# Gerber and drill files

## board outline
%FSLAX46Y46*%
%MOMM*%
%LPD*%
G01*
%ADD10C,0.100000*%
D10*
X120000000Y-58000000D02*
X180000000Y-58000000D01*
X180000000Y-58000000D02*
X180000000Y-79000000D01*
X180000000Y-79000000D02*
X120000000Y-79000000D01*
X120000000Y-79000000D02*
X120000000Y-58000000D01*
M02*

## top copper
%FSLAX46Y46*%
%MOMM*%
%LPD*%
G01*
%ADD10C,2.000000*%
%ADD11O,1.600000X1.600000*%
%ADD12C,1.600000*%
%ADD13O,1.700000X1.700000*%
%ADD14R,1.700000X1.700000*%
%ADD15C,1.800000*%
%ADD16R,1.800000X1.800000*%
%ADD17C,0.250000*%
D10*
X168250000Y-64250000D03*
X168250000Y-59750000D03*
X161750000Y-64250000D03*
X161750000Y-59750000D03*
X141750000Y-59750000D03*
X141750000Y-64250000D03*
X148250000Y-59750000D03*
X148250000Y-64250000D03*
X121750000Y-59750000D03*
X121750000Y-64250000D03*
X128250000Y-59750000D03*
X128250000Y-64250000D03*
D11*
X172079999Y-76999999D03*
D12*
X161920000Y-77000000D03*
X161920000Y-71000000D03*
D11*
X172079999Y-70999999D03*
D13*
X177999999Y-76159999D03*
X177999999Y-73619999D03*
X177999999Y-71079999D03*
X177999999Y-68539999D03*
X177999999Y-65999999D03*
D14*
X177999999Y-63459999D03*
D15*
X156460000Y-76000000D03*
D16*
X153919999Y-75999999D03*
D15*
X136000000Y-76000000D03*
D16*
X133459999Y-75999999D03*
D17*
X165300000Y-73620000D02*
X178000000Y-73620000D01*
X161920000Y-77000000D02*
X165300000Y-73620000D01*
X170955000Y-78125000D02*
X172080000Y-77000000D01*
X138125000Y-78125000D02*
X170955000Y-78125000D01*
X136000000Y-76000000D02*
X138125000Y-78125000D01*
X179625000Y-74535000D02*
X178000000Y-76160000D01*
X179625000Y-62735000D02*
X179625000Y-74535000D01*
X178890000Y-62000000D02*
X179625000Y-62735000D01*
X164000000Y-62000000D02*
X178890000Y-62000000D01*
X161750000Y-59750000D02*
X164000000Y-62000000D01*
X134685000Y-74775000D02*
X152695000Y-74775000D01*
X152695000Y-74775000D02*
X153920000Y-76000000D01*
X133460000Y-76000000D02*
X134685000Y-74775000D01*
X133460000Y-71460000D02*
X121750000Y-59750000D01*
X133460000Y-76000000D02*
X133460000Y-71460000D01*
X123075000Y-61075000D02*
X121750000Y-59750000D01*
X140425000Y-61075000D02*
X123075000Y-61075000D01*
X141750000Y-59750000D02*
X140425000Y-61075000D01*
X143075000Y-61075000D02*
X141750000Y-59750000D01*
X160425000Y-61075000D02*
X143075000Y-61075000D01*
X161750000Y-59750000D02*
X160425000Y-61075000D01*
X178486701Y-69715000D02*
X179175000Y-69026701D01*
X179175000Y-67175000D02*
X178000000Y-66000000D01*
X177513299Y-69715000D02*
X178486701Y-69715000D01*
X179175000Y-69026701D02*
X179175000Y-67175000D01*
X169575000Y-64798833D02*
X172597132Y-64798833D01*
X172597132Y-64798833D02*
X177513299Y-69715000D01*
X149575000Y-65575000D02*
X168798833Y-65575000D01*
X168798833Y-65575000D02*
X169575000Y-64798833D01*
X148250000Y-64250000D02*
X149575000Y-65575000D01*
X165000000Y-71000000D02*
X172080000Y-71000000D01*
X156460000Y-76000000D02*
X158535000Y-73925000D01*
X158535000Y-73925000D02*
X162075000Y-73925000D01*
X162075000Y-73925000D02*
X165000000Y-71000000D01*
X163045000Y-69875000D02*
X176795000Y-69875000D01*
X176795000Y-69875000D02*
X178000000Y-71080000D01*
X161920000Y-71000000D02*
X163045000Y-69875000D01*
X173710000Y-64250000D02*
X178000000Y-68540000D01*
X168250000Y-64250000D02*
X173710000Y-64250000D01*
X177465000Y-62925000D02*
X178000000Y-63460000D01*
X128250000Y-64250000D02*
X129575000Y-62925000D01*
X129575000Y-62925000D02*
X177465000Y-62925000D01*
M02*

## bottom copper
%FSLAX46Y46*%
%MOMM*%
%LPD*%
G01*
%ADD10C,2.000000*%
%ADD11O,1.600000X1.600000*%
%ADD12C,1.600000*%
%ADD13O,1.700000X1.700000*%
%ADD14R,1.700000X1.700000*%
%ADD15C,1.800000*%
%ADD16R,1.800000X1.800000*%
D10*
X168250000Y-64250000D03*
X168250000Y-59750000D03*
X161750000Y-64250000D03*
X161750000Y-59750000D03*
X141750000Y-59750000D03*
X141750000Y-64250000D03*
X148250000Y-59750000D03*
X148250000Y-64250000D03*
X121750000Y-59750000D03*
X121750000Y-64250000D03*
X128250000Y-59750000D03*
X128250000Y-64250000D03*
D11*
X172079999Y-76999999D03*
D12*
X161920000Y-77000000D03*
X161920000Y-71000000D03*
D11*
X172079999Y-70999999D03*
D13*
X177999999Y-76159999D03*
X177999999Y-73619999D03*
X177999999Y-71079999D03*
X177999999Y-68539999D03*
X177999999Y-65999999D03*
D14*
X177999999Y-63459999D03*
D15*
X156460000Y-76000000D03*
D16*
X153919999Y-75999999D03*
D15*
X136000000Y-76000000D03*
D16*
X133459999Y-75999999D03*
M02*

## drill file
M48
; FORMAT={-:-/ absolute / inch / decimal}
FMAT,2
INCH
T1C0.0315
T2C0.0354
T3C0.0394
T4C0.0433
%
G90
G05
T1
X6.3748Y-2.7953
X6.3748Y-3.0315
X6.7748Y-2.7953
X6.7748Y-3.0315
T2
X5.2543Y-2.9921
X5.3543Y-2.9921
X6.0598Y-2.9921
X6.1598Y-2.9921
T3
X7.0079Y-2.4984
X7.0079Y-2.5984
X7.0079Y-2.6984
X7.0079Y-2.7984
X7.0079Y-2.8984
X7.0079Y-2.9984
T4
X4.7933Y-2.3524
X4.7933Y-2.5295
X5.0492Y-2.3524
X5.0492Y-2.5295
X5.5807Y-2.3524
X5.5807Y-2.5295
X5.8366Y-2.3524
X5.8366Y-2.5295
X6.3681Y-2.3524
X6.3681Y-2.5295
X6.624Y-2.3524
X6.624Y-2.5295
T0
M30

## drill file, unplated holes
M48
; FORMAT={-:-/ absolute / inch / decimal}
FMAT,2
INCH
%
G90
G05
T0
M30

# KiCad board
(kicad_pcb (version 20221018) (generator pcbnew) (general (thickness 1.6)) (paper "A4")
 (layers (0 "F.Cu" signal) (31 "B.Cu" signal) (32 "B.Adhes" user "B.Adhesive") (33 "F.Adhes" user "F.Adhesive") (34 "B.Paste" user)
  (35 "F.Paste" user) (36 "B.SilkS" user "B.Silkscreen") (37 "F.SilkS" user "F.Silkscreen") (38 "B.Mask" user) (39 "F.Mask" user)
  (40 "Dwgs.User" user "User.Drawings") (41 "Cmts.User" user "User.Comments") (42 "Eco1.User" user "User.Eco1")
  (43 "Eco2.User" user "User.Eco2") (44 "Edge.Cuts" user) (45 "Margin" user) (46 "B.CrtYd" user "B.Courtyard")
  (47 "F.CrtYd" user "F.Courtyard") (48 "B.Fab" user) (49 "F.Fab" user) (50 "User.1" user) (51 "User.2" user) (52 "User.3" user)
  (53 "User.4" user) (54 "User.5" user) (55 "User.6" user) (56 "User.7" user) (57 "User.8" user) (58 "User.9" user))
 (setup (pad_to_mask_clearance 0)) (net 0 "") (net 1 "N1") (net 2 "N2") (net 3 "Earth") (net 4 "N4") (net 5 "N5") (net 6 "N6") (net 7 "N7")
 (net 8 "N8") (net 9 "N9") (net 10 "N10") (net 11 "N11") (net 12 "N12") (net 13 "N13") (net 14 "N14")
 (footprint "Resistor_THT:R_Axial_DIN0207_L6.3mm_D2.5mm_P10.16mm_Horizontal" (layer "F.Cu") (at 161.92 77)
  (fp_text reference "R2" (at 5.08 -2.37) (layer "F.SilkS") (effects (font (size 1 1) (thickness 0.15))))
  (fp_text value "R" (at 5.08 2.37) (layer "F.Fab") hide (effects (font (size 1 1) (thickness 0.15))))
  (pad "1" thru_hole circle (at 0 0) (size 1.6 1.6) (drill 0.8) (layers "*.Cu" "*.Mask") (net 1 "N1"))
  (pad "2" thru_hole oval (at 10.16 0) (size 1.6 1.6) (drill 0.8) (layers "*.Cu" "*.Mask") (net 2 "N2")))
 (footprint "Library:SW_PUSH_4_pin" (layer "F.Cu") (at 161.75 59.75)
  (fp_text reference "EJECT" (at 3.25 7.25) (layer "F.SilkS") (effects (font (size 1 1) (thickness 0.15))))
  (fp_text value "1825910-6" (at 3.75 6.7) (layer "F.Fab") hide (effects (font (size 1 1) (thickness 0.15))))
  (pad "1" thru_hole circle (at 0 0 90) (size 2 2) (drill 1.1) (layers "*.Cu" "*.Mask") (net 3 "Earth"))
  (pad "2" thru_hole circle (at 0 4.5 90) (size 2 2) (drill 1.1) (layers "*.Cu" "*.Mask") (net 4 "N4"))
  (pad "3" thru_hole circle (at 6.5 0 90) (size 2 2) (drill 1.1) (layers "*.Cu" "*.Mask") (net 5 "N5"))
  (pad "4" thru_hole circle (at 6.5 4.5 90) (size 2 2) (drill 1.1) (layers "*.Cu" "*.Mask") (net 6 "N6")))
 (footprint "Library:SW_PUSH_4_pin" (layer "F.Cu") (at 141.75 59.75)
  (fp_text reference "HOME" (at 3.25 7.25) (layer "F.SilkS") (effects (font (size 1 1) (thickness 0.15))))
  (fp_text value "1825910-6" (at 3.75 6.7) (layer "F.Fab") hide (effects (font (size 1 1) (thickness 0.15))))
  (pad "1" thru_hole circle (at 0 0 90) (size 2 2) (drill 1.1) (layers "*.Cu" "*.Mask") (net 3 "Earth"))
  (pad "2" thru_hole circle (at 0 4.5 90) (size 2 2) (drill 1.1) (layers "*.Cu" "*.Mask") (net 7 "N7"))
  (pad "3" thru_hole circle (at 6.5 0 90) (size 2 2) (drill 1.1) (layers "*.Cu" "*.Mask") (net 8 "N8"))
  (pad "4" thru_hole circle (at 6.5 4.5 90) (size 2 2) (drill 1.1) (layers "*.Cu" "*.Mask") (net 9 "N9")))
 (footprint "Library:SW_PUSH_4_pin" (layer "F.Cu") (at 121.75 59.75)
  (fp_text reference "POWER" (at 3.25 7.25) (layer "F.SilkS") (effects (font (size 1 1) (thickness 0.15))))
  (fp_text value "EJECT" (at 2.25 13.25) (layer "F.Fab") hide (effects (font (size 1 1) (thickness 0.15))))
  (pad "1" thru_hole circle (at 0 0 90) (size 2 2) (drill 1.1) (layers "*.Cu" "*.Mask") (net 3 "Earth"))
  (pad "2" thru_hole circle (at 0 4.5 90) (size 2 2) (drill 1.1) (layers "*.Cu" "*.Mask") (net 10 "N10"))
  (pad "3" thru_hole circle (at 6.5 0 90) (size 2 2) (drill 1.1) (layers "*.Cu" "*.Mask") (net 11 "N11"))
  (pad "4" thru_hole circle (at 6.5 4.5 90) (size 2 2) (drill 1.1) (layers "*.Cu" "*.Mask") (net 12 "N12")))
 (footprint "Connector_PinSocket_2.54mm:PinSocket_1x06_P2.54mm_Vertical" (layer "F.Cu") (at 178 63.46)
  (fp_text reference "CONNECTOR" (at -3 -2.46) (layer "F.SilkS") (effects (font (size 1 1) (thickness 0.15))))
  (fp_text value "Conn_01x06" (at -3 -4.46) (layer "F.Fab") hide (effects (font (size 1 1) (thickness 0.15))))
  (pad "1" thru_hole rect (at 0 0) (size 1.7 1.7) (drill 1) (layers "*.Cu" "*.Mask") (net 12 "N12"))
  (pad "2" thru_hole oval (at 0 2.54) (size 1.7 1.7) (drill 1) (layers "*.Cu" "*.Mask") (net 9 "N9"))
  (pad "3" thru_hole oval (at 0 5.08) (size 1.7 1.7) (drill 1) (layers "*.Cu" "*.Mask") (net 6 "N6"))
  (pad "4" thru_hole oval (at 0 7.62) (size 1.7 1.7) (drill 1) (layers "*.Cu" "*.Mask") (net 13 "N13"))
  (pad "5" thru_hole oval (at 0 10.16) (size 1.7 1.7) (drill 1) (layers "*.Cu" "*.Mask") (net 1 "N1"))
  (pad "6" thru_hole oval (at 0 12.7) (size 1.7 1.7) (drill 1) (layers "*.Cu" "*.Mask") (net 3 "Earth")))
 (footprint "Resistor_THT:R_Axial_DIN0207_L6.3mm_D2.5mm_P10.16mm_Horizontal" (layer "F.Cu") (at 161.92 71)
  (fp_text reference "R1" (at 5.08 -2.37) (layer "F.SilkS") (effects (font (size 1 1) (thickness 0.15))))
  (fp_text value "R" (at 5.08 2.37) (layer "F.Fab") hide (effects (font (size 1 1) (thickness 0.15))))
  (pad "1" thru_hole circle (at 0 0) (size 1.6 1.6) (drill 0.8) (layers "*.Cu" "*.Mask") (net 13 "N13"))
  (pad "2" thru_hole oval (at 10.16 0) (size 1.6 1.6) (drill 0.8) (layers "*.Cu" "*.Mask") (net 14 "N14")))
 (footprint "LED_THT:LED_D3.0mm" (layer "F.Cu") (at 133.46 76)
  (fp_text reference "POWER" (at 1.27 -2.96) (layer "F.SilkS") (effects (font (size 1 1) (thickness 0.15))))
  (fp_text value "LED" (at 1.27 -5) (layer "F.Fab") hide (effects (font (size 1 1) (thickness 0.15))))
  (pad "1" thru_hole rect (at 0 0) (size 1.8 1.8) (drill 0.9) (layers "*.Cu" "*.Mask") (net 3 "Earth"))
  (pad "2" thru_hole circle (at 2.54 0) (size 1.8 1.8) (drill 0.9) (layers "*.Cu" "*.Mask") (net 2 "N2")))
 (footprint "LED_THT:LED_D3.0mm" (layer "F.Cu") (at 153.92 76)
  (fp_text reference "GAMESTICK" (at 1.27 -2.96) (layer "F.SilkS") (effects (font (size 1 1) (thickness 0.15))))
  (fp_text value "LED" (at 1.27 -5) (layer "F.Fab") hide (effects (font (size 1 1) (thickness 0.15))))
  (pad "1" thru_hole rect (at 0 0) (size 1.8 1.8) (drill 0.9) (layers "*.Cu" "*.Mask") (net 3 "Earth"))
  (pad "2" thru_hole circle (at 2.54 0) (size 1.8 1.8) (drill 0.9) (layers "*.Cu" "*.Mask") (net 14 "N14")))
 (gr_rect (start 120 58) (end 180 79) (stroke (width 0.1) (type default)) (fill none) (layer "Edge.Cuts"))
 (segment (start 152.695 74.775) (end 153.92 76) (width 0.25) (layer "F.Cu") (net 3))
 (segment (start 123.075 61.075) (end 121.75 59.75) (width 0.25) (layer "F.Cu") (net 3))
 (segment (start 133.46 76) (end 133.46 71.46) (width 0.25) (layer "F.Cu") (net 3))
 (segment (start 161.75 59.75) (end 160.425 61.075) (width 0.25) (layer "F.Cu") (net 3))
 (segment (start 133.46 76) (end 134.685 74.775) (width 0.25) (layer "F.Cu") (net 3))
 (segment (start 143.075 61.075) (end 141.75 59.75) (width 0.25) (layer "F.Cu") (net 3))
 (segment (start 160.425 61.075) (end 143.075 61.075) (width 0.25) (layer "F.Cu") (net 3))
 (segment (start 164 62) (end 178.89 62) (width 0.25) (layer "F.Cu") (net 3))
 (segment (start 161.75 59.75) (end 164 62) (width 0.25) (layer "F.Cu") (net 3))
 (segment (start 133.46 71.46) (end 121.75 59.75) (width 0.25) (layer "F.Cu") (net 3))
 (segment (start 179.625 62.735) (end 179.625 74.535) (width 0.25) (layer "F.Cu") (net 3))
 (segment (start 134.685 74.775) (end 152.695 74.775) (width 0.25) (layer "F.Cu") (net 3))
 (segment (start 140.425 61.075) (end 123.075 61.075) (width 0.25) (layer "F.Cu") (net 3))
 (segment (start 178.89 62) (end 179.625 62.735) (width 0.25) (layer "F.Cu") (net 3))
 (segment (start 141.75 59.75) (end 140.425 61.075) (width 0.25) (layer "F.Cu") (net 3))
 (segment (start 179.625 74.535) (end 178 76.16) (width 0.25) (layer "F.Cu") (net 3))
 (segment (start 138.125 78.125) (end 170.955 78.125) (width 0.25) (layer "F.Cu") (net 2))
 (segment (start 136 76) (end 138.125 78.125) (width 0.25) (layer "F.Cu") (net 2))
 (segment (start 170.955 78.125) (end 172.08 77) (width 0.25) (layer "F.Cu") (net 2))
 (segment (start 156.46 76) (end 158.535 73.925) (width 0.25) (layer "F.Cu") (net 14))
 (segment (start 162.075 73.925) (end 165 71) (width 0.25) (layer "F.Cu") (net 14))
 (segment (start 165 71) (end 172.08 71) (width 0.25) (layer "F.Cu") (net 14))
 (segment (start 158.535 73.925) (end 162.075 73.925) (width 0.25) (layer "F.Cu") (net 14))
 (segment (start 128.25 64.25) (end 129.575 62.925) (width 0.25) (layer "F.Cu") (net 12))
 (segment (start 129.575 62.925) (end 177.465 62.925) (width 0.25) (layer "F.Cu") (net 12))
 (segment (start 177.465 62.925) (end 178 63.46) (width 0.25) (layer "F.Cu") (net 12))
 (segment (start 179.175 69.026701) (end 179.175 67.175) (width 0.25) (layer "F.Cu") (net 9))
 (segment (start 148.25 64.25) (end 149.575 65.575) (width 0.25) (layer "F.Cu") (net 9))
 (segment (start 168.798833 65.575) (end 169.575 64.798833) (width 0.25) (layer "F.Cu") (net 9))
 (segment (start 177.513299 69.715) (end 178.486701 69.715) (width 0.25) (layer "F.Cu") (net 9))
 (segment (start 178.486701 69.715) (end 179.175 69.026701) (width 0.25) (layer "F.Cu") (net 9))
 (segment (start 169.575 64.798833) (end 172.597132 64.798833) (width 0.25) (layer "F.Cu") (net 9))
 (segment (start 179.175 67.175) (end 178 66) (width 0.25) (layer "F.Cu") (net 9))
 (segment (start 172.597132 64.798833) (end 177.513299 69.715) (width 0.25) (layer "F.Cu") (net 9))
 (segment (start 149.575 65.575) (end 168.798833 65.575) (width 0.25) (layer "F.Cu") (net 9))
 (segment (start 173.71 64.25) (end 178 68.54) (width 0.25) (layer "F.Cu") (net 6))
 (segment (start 168.25 64.25) (end 173.71 64.25) (width 0.25) (layer "F.Cu") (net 6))
 (segment (start 161.92 71) (end 163.045 69.875) (width 0.25) (layer "F.Cu") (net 13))
 (segment (start 176.795 69.875) (end 178 71.08) (width 0.25) (layer "F.Cu") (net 13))
 (segment (start 163.045 69.875) (end 176.795 69.875) (width 0.25) (layer "F.Cu") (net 13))
 (segment (start 161.92 77) (end 165.3 73.62) (width 0.25) (layer "F.Cu") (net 1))
 (segment (start 165.3 73.62) (end 178 73.62) (width 0.25) (layer "F.Cu") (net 1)))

